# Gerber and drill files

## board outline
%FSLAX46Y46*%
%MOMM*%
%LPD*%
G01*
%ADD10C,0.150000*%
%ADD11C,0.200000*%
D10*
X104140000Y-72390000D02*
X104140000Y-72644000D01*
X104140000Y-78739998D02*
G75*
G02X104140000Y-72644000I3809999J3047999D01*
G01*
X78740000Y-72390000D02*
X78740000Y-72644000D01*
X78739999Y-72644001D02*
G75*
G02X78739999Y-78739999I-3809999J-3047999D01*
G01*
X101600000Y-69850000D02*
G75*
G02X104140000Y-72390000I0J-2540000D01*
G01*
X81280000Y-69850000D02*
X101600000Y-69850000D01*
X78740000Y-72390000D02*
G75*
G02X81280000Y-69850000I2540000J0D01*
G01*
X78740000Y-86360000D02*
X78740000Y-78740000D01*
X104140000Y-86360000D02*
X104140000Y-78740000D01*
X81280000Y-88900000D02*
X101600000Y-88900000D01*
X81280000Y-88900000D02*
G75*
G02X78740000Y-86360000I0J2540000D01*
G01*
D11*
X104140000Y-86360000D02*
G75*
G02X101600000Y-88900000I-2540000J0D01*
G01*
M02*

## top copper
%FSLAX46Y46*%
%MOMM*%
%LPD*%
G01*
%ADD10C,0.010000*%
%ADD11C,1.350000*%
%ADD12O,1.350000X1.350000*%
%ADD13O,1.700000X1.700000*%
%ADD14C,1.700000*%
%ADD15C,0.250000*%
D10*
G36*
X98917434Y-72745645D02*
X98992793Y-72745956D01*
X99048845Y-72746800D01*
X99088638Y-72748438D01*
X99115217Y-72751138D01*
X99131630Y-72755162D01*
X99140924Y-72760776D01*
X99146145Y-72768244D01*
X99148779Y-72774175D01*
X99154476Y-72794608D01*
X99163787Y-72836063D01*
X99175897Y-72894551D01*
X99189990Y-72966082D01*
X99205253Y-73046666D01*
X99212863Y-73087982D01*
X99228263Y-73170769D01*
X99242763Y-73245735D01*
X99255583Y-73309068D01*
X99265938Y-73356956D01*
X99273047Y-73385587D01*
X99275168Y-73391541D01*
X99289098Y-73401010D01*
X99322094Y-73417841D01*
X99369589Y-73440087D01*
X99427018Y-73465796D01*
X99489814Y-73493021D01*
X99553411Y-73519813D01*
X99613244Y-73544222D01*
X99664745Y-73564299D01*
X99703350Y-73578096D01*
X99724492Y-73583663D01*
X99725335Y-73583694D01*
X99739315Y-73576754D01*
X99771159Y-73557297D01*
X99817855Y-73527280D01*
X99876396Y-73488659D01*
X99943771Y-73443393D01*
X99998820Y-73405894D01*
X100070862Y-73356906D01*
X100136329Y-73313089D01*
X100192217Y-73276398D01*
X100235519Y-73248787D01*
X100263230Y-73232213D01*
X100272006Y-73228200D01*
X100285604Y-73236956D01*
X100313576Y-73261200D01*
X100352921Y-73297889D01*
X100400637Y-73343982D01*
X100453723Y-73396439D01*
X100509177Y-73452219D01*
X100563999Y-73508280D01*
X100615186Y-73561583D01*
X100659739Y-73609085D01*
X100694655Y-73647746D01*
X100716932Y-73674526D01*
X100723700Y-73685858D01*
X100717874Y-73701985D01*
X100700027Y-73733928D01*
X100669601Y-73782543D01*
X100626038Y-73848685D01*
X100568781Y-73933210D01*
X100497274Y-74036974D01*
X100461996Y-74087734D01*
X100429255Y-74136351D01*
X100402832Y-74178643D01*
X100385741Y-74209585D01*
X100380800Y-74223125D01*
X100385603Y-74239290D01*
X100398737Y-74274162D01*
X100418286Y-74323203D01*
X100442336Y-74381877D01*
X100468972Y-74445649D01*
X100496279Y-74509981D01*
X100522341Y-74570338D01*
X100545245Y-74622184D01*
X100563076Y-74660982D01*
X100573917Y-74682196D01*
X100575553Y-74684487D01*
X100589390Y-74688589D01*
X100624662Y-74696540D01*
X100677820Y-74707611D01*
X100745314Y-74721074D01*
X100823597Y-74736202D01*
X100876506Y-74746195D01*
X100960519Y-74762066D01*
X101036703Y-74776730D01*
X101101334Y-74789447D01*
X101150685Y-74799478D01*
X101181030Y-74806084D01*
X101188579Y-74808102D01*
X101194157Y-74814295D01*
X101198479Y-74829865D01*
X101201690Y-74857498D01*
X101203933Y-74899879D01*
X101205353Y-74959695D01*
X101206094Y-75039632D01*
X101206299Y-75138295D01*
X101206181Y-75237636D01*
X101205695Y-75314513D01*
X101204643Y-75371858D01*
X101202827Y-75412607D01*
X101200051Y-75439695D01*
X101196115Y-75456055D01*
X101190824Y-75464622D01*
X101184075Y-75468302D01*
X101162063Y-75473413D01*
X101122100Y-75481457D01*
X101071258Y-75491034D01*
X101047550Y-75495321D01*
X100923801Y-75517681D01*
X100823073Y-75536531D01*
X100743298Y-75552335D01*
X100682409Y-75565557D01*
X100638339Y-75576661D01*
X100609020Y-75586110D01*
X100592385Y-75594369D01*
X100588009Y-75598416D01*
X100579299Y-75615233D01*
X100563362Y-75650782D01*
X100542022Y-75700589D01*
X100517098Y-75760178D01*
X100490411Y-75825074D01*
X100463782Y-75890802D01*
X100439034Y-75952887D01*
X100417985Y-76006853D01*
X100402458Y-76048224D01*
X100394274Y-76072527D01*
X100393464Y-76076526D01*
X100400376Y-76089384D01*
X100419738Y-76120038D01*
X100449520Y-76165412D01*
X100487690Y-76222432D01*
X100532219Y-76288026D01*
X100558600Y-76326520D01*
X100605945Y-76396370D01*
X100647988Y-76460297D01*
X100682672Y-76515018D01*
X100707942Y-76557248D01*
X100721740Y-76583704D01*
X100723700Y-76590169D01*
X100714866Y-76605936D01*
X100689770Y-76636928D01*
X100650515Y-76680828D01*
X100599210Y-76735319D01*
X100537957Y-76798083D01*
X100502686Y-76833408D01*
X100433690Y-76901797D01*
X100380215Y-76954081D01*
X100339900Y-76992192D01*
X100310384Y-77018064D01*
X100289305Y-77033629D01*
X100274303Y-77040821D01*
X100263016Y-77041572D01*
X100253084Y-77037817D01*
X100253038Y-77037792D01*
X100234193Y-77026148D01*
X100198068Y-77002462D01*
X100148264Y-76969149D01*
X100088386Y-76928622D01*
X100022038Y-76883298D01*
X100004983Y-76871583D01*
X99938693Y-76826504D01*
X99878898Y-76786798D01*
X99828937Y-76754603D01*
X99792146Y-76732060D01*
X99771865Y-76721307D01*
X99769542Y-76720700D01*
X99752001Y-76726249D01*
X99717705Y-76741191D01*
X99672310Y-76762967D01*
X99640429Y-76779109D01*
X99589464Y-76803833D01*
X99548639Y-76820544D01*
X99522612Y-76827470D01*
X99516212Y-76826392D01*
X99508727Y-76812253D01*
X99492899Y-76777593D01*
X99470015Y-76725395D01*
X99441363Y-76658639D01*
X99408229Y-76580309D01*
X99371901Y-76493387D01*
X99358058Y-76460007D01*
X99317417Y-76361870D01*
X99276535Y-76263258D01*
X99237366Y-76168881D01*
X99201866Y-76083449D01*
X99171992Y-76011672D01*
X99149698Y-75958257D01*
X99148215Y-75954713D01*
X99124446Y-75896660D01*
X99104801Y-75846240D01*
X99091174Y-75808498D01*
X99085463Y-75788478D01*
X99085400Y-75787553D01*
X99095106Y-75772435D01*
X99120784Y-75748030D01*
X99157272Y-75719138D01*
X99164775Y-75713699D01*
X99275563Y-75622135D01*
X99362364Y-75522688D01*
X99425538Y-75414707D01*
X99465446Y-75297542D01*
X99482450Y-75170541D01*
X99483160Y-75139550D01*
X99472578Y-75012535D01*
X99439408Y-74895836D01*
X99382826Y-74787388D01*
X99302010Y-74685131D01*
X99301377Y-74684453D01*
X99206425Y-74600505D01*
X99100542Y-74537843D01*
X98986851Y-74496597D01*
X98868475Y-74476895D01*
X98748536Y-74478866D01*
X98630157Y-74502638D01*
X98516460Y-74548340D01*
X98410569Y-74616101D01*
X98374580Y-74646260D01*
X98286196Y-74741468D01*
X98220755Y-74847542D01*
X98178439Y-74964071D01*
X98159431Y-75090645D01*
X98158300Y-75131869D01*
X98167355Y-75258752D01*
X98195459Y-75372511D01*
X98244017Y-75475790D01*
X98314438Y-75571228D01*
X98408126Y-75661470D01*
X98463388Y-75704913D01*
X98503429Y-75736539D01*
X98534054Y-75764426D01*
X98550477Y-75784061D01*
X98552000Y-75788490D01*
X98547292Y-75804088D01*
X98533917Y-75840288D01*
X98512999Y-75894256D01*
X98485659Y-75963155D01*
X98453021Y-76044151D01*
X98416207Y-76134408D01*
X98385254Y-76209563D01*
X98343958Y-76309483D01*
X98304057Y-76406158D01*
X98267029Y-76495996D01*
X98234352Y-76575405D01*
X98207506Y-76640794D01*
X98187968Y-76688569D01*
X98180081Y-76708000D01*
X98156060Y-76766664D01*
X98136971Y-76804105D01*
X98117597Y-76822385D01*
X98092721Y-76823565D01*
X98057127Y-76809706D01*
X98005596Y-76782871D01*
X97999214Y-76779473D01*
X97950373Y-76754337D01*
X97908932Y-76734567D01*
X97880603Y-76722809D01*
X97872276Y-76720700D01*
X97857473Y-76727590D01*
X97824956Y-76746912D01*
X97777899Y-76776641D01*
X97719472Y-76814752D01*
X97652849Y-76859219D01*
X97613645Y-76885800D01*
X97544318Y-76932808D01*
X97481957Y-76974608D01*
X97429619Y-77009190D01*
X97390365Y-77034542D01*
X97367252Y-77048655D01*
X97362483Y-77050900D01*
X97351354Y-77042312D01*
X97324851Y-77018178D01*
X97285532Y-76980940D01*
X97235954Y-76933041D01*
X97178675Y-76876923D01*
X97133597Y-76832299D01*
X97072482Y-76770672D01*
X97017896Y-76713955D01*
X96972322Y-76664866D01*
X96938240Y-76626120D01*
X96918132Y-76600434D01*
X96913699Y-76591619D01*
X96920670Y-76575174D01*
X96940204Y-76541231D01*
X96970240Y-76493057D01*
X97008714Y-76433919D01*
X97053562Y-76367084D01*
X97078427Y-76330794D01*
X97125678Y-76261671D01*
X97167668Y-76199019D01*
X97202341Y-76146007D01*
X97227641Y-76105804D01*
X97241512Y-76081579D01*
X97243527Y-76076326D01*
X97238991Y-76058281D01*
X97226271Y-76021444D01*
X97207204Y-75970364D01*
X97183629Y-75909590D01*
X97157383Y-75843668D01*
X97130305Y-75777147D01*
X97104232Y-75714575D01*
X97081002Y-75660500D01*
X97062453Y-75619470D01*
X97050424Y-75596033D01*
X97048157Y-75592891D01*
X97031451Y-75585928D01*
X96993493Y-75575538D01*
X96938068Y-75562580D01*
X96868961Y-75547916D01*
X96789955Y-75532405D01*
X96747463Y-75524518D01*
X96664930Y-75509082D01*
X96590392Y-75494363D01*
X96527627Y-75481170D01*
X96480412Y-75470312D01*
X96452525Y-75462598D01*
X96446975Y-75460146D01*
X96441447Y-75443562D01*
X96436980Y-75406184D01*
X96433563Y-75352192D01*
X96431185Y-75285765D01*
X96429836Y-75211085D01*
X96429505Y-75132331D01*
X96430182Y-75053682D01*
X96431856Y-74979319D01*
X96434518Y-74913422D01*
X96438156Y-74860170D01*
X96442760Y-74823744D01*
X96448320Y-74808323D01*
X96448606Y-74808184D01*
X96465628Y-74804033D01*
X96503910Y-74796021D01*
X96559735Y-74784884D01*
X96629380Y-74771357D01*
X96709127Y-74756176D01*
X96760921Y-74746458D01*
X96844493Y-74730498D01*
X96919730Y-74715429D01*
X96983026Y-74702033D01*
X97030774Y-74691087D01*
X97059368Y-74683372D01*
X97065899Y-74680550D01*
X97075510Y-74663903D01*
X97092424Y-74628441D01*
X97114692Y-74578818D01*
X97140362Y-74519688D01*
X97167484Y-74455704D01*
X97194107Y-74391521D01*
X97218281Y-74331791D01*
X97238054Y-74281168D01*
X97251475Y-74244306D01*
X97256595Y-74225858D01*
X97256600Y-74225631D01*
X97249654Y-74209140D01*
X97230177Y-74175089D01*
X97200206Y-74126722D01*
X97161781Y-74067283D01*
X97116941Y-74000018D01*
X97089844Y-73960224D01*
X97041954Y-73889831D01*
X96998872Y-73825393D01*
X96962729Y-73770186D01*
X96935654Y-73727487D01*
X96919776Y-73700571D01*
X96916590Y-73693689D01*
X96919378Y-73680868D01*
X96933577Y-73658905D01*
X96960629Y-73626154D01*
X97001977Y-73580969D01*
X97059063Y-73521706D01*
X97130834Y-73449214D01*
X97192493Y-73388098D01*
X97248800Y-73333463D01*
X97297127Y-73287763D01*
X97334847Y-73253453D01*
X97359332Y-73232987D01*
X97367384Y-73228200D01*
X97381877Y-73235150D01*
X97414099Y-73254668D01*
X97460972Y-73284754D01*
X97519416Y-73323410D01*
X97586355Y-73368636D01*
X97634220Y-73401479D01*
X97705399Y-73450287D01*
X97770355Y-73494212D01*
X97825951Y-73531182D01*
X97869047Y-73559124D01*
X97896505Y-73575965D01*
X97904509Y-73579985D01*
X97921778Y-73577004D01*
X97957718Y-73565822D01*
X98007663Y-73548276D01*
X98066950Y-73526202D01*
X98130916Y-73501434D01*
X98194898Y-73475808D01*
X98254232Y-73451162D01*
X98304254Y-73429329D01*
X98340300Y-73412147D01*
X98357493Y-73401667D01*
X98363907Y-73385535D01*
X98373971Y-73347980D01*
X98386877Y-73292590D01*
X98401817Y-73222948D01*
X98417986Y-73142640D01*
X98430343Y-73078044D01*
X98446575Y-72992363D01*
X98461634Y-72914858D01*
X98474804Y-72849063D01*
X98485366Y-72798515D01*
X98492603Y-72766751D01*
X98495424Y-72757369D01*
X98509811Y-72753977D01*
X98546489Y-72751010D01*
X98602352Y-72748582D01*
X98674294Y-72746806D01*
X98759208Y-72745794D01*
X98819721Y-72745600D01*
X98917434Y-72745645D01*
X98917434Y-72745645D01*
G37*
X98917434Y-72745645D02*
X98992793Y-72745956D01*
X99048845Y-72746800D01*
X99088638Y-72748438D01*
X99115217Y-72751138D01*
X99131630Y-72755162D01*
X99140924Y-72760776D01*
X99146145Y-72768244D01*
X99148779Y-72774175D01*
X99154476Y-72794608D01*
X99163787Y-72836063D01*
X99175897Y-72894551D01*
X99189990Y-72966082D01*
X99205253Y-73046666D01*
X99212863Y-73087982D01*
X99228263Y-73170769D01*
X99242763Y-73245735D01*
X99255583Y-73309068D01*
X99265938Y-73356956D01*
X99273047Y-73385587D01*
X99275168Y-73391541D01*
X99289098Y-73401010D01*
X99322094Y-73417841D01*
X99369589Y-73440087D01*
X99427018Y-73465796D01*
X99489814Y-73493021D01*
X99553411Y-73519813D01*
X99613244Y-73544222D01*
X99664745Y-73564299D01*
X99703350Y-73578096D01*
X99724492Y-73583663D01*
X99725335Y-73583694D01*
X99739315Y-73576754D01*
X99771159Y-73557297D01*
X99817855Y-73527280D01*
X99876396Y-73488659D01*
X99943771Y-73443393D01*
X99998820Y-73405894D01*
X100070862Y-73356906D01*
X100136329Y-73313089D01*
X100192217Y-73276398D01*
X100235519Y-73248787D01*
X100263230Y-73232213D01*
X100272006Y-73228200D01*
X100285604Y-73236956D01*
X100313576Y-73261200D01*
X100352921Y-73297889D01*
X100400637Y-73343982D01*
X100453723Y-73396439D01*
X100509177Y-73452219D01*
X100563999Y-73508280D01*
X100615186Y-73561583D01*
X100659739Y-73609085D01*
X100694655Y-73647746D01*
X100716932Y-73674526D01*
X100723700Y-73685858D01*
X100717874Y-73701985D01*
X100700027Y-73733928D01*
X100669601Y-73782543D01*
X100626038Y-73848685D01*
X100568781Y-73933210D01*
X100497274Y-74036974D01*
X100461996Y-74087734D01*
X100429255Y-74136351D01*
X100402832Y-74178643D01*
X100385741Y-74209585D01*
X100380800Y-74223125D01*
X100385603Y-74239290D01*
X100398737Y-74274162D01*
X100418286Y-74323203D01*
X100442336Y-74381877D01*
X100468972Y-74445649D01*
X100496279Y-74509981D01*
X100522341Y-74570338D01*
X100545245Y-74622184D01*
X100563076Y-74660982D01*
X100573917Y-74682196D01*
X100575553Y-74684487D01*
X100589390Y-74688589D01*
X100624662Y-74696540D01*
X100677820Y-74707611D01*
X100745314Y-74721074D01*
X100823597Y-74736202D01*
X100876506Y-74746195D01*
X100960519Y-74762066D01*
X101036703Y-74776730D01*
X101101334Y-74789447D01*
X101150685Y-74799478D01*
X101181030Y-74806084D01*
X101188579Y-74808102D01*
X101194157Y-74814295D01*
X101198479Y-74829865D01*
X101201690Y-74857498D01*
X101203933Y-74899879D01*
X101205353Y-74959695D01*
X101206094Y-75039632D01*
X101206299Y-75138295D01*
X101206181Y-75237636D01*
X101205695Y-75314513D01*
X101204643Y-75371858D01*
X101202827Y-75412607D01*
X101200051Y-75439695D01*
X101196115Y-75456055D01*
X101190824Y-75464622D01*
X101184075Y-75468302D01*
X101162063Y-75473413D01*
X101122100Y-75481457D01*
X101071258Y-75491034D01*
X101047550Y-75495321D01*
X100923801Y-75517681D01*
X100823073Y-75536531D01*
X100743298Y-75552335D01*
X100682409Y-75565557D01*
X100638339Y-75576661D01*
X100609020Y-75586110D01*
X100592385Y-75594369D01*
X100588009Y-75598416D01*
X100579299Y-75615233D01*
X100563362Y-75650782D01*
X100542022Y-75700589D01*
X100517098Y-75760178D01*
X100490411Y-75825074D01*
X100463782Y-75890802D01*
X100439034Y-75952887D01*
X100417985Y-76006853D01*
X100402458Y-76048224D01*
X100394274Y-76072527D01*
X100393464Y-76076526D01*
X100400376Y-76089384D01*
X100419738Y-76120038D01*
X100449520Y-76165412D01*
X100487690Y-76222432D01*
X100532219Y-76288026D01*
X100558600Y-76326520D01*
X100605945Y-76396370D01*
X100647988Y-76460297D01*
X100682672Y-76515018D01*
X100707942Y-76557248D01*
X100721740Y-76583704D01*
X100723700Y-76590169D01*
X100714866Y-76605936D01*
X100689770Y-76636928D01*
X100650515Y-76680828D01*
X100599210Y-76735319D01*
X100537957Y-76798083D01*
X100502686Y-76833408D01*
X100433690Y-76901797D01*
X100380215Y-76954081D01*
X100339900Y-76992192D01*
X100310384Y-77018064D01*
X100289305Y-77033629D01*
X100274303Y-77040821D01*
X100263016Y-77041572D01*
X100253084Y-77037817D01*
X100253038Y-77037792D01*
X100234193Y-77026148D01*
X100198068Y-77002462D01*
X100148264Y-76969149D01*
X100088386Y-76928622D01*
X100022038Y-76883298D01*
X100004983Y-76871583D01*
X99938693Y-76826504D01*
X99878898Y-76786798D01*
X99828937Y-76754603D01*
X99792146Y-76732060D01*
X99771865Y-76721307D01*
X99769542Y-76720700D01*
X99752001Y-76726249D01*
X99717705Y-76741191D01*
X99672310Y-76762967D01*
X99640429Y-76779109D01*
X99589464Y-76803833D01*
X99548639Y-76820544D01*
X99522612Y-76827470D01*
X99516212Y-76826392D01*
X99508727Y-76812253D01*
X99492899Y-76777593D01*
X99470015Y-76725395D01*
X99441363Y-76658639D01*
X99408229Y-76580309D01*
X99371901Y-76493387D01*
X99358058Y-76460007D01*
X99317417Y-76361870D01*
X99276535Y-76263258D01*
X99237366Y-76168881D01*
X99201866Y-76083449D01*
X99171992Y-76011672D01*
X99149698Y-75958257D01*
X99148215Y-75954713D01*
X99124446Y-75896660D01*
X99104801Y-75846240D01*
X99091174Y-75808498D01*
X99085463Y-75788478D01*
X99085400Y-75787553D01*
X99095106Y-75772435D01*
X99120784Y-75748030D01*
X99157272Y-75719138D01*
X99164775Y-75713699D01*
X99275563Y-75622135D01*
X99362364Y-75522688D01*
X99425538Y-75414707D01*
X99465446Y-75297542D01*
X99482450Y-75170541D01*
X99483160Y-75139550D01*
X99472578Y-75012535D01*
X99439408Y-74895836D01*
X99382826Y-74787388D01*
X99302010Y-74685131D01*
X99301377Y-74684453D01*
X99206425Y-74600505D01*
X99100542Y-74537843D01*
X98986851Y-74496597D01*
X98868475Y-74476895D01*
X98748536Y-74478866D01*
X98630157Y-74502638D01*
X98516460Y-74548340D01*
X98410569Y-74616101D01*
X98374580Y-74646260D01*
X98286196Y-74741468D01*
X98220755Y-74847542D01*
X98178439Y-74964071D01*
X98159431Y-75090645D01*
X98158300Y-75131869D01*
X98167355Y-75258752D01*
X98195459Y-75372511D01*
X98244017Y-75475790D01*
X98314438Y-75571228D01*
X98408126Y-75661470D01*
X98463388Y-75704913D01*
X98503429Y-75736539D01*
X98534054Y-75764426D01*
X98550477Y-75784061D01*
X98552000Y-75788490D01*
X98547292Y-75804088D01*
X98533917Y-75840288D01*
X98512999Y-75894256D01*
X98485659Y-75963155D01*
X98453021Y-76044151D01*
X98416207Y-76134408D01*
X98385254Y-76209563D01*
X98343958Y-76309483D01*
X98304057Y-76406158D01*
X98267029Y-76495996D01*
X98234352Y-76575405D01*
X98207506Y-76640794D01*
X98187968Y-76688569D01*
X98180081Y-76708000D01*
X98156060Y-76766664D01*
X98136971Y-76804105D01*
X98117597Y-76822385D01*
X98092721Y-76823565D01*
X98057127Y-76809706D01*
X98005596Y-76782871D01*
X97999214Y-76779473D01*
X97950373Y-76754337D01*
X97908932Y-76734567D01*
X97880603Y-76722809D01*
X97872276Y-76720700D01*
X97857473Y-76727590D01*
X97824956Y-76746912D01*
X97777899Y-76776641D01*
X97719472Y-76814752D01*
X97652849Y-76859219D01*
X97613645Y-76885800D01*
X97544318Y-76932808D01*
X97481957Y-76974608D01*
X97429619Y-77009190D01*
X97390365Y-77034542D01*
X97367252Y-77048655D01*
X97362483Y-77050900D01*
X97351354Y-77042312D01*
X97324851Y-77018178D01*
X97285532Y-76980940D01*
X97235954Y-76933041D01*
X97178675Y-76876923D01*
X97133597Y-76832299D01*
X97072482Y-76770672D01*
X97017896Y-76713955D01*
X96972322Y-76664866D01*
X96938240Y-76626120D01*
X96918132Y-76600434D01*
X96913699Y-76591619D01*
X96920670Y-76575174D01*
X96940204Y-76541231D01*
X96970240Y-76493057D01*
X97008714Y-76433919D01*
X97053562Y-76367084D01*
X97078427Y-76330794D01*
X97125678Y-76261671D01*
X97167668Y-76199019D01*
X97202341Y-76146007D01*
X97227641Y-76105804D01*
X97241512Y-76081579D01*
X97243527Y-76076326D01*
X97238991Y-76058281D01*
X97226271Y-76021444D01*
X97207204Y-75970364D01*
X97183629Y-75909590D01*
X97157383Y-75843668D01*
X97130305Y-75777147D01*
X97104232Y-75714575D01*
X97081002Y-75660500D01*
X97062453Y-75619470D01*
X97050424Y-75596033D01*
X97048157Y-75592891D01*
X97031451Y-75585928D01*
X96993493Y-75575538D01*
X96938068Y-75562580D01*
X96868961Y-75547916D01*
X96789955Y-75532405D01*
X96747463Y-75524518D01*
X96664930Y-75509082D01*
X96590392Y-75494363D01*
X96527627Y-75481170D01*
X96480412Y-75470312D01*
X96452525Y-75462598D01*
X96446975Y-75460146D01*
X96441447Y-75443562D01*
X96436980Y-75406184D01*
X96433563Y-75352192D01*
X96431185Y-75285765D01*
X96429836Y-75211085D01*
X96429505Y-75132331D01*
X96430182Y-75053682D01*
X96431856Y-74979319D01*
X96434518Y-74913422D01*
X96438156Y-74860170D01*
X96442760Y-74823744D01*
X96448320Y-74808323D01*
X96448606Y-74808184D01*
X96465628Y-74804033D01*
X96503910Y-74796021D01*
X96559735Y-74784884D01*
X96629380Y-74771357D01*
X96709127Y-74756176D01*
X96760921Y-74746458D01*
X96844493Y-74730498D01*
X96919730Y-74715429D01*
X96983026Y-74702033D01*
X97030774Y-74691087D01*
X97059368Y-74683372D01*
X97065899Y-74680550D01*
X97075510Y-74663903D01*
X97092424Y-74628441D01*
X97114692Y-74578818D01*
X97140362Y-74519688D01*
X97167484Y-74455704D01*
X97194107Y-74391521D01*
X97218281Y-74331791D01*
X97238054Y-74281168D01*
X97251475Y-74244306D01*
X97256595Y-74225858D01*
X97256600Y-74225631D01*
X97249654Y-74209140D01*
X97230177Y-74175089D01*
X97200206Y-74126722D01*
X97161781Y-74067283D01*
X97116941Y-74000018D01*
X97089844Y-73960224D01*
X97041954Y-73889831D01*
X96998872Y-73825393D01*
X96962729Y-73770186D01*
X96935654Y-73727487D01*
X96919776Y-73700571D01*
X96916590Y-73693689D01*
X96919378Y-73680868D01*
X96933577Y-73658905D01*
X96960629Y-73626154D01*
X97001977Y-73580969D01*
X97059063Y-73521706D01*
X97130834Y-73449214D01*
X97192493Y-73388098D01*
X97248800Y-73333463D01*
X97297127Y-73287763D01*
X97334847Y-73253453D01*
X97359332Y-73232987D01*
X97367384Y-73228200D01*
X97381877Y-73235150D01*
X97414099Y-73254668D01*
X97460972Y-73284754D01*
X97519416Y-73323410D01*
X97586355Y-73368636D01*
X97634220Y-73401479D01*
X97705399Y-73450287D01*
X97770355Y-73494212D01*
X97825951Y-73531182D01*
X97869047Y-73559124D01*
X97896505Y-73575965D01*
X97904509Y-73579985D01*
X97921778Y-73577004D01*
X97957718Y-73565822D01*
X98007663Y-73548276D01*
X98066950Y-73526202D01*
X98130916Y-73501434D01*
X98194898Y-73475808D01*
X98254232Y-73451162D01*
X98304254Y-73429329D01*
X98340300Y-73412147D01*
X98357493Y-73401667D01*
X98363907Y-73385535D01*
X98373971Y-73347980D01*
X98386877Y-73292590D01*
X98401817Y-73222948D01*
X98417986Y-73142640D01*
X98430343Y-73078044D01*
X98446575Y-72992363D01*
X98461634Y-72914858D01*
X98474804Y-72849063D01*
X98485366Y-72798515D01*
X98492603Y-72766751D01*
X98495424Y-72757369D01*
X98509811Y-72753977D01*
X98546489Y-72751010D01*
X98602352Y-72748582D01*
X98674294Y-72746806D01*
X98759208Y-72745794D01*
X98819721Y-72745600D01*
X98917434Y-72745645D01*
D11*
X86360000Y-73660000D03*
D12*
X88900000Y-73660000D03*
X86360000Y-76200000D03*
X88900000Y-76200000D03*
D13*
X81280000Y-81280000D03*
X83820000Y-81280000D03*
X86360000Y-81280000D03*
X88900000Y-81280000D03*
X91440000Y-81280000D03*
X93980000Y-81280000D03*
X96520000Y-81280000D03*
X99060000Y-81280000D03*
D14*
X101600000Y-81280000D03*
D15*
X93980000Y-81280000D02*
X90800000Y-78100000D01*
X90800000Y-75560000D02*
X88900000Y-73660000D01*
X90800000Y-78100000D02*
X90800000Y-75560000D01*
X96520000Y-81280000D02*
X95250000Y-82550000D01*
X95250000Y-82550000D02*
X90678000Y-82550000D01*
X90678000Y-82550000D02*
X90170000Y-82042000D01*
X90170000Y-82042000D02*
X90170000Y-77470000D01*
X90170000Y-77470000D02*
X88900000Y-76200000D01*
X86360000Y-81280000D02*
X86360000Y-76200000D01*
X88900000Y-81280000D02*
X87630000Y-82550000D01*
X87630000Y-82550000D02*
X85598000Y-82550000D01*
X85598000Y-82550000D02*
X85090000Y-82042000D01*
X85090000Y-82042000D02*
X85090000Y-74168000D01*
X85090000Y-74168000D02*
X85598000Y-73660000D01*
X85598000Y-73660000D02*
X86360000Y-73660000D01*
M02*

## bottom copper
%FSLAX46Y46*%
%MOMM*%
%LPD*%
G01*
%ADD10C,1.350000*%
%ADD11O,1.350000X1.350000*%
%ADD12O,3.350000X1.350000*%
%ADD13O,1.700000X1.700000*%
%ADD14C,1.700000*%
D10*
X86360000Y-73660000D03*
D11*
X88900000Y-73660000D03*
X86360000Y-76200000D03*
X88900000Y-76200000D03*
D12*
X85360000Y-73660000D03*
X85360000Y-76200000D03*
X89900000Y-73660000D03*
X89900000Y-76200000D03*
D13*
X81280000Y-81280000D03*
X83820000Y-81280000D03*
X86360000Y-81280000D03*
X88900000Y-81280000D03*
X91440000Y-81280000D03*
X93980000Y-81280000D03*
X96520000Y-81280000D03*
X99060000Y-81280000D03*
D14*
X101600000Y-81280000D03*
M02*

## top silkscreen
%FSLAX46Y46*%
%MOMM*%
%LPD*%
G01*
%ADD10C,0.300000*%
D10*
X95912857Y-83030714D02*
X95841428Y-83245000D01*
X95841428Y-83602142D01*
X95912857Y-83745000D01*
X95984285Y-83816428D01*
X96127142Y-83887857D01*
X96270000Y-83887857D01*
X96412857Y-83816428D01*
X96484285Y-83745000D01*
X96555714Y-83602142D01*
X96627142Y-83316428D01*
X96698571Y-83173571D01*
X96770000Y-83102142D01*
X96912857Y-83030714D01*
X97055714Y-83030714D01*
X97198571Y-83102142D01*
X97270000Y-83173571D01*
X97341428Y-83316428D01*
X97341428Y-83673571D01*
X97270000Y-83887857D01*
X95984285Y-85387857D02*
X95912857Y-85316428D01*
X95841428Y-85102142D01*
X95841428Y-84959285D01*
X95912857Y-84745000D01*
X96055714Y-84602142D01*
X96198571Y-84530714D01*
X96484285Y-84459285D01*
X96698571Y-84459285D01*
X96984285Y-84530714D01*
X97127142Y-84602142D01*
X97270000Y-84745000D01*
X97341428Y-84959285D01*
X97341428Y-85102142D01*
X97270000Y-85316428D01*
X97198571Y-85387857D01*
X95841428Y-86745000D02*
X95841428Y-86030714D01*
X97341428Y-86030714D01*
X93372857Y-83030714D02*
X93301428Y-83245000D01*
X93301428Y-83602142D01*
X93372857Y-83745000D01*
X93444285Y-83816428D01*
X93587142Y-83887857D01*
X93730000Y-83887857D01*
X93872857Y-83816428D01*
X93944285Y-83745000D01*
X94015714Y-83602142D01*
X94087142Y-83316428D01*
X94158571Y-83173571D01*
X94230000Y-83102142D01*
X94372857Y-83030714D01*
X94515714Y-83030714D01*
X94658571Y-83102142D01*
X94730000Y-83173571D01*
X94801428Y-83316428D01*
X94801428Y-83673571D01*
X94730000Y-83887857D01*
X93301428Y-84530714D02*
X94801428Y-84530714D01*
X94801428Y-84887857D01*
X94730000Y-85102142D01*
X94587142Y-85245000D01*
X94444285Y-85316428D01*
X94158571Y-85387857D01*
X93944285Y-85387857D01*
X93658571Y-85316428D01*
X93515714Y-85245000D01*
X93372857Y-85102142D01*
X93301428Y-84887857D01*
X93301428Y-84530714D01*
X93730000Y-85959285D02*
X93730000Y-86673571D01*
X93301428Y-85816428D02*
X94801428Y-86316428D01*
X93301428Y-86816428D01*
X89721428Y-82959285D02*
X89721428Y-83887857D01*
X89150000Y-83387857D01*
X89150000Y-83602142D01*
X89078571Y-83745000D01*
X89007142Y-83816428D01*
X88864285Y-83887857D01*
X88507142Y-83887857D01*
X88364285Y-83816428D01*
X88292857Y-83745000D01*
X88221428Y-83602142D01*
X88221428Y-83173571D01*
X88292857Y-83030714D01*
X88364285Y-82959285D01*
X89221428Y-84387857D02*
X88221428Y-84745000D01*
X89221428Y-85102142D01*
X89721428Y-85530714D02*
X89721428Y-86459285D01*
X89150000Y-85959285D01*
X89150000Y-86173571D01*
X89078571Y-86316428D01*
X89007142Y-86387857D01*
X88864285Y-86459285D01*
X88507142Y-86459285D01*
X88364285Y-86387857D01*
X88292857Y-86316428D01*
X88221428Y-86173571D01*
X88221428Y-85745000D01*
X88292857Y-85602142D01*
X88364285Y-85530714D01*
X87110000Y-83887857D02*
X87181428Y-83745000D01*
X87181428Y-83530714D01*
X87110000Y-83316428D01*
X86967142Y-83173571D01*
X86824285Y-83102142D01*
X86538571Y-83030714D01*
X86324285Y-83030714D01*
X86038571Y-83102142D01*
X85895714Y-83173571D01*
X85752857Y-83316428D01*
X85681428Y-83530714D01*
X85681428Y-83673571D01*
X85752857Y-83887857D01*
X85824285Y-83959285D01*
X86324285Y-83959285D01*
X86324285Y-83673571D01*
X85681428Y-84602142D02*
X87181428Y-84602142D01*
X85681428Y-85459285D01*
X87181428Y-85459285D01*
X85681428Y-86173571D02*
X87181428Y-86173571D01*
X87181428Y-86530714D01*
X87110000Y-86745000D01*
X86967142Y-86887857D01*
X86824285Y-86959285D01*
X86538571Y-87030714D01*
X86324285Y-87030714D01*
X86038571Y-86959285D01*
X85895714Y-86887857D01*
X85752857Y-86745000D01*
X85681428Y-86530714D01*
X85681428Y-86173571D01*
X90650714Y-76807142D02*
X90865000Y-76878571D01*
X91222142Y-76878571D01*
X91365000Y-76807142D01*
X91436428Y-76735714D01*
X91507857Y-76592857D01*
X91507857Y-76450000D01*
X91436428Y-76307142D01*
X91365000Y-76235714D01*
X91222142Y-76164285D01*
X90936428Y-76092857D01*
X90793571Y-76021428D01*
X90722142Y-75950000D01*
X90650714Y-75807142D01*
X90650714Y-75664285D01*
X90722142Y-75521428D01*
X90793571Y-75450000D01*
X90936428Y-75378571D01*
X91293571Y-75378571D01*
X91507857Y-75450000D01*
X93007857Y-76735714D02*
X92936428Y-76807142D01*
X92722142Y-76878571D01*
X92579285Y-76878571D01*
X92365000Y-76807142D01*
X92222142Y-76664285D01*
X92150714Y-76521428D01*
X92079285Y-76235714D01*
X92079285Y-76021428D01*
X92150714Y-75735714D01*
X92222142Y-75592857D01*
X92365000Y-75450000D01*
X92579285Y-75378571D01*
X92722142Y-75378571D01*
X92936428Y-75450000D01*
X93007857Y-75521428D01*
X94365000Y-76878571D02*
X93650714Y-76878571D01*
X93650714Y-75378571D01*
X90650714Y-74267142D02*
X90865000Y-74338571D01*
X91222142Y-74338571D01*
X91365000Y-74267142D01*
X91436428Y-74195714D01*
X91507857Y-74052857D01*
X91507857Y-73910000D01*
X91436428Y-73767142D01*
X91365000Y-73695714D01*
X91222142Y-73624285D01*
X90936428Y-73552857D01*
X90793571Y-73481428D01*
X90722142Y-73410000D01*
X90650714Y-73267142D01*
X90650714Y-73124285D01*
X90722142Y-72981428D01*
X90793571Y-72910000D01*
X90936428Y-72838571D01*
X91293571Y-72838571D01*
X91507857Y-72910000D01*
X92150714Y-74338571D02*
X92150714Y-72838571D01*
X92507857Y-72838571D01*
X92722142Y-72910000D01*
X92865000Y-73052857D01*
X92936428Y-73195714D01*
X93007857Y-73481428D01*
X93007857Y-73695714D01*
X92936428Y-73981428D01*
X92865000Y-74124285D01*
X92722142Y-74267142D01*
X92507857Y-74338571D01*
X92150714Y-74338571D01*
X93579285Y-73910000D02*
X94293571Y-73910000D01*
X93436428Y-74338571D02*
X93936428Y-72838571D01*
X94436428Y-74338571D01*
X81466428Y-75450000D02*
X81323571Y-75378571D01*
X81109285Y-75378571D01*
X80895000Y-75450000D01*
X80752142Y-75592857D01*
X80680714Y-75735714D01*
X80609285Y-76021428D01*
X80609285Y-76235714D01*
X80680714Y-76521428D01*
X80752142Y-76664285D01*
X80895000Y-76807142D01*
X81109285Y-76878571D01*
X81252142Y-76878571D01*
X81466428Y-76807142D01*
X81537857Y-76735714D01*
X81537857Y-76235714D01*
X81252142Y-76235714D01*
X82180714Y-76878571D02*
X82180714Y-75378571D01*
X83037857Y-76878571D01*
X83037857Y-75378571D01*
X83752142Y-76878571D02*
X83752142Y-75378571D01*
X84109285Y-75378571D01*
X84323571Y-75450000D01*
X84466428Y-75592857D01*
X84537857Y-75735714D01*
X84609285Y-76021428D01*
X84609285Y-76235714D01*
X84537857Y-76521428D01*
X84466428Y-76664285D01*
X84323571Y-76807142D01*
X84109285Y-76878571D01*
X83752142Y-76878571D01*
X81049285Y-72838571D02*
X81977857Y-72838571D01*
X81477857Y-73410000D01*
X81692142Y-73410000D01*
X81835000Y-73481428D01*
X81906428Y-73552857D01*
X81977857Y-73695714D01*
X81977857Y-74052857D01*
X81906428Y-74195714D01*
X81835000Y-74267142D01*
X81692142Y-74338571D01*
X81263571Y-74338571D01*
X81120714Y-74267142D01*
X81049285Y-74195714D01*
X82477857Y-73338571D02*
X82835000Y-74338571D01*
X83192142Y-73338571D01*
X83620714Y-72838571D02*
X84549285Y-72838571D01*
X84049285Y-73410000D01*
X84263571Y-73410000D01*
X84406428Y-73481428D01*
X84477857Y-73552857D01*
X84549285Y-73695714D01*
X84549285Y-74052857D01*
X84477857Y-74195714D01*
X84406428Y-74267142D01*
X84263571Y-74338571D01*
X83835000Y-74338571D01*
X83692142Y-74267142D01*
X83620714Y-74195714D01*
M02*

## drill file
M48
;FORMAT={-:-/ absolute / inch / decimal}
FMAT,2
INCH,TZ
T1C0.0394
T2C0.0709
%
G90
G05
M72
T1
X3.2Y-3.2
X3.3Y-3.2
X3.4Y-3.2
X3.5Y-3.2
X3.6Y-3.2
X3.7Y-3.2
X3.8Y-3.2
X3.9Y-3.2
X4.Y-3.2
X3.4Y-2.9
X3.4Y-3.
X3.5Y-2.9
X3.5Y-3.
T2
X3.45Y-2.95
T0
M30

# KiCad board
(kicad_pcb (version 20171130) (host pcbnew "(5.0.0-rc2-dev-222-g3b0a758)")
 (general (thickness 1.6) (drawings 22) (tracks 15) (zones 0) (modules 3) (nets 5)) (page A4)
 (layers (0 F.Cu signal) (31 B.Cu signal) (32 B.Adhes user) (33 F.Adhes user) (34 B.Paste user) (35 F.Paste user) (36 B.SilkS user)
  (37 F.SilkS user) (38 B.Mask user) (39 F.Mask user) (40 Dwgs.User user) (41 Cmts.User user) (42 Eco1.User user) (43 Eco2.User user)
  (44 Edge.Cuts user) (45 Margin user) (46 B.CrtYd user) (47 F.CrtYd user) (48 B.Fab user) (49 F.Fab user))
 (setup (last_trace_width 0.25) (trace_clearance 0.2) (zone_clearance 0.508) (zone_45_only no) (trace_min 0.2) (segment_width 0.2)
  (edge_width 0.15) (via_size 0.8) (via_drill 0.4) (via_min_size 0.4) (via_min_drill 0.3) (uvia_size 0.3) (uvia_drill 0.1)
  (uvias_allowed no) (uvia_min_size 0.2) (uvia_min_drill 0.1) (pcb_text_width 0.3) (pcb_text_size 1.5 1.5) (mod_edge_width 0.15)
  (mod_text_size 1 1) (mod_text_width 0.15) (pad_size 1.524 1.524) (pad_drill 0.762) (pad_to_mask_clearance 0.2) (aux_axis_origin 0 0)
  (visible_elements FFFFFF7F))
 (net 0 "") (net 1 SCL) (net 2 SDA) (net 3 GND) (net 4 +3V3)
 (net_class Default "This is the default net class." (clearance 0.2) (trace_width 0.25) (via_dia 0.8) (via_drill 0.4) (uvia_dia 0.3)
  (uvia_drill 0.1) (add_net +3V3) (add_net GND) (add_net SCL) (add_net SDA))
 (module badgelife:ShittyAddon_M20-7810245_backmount (layer F.Cu) (at 86.36 73.66)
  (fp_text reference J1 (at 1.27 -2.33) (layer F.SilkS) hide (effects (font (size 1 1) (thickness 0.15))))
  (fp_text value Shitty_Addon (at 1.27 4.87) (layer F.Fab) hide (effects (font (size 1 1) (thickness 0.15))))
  (pad "" np_thru_hole circle (at 1.27 1.27) (size 1.8 1.8) (drill 1.8) (layers *.Cu *.Mask) (solder_mask_margin 0.001))
  (pad 3 smd oval (at 2.54 2.54) (size 3.35 1.35) (drill (offset 1 0)) (layers B.Cu B.Paste B.Mask) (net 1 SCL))
  (pad 4 smd oval (at 2.54 0) (size 3.35 1.35) (drill (offset 1 0)) (layers B.Cu B.Paste B.Mask) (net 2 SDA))
  (pad 2 smd oval (at 0 2.54) (size 3.35 1.35) (drill (offset -1 0)) (layers B.Cu B.Paste B.Mask) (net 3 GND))
  (pad 1 smd oval (at 0 0) (size 3.35 1.35) (drill (offset -1 0)) (layers B.Cu B.Paste B.Mask) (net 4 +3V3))
  (pad 3 thru_hole oval (at 2.54 2.54) (size 1.35 1.35) (drill 1) (layers *.Cu *.Mask) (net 1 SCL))
  (pad 2 thru_hole oval (at 0 2.54) (size 1.35 1.35) (drill 1) (layers *.Cu *.Mask) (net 3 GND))
  (pad 4 thru_hole oval (at 2.54 0) (size 1.35 1.35) (drill 1) (layers *.Cu *.Mask) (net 2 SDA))
  (pad 1 thru_hole circle (at 0 0) (size 1.35 1.35) (drill 1) (layers *.Cu *.Mask) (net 4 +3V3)))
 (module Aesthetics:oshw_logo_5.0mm (layer F.Cu) (at 98.806 74.93)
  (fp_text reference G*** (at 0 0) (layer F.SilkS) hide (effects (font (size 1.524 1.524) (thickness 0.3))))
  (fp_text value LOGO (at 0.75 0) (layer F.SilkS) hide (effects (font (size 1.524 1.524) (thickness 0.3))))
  (fp_poly
   (pts (xy 0.111434 -2.184355) (xy 0.186793 -2.184044) (xy 0.242845 -2.1832) (xy 0.282638 -2.181562) (xy 0.309217 -2.178862)
    (xy 0.32563 -2.174838) (xy 0.334924 -2.169224) (xy 0.340145 -2.161756) (xy 0.342779 -2.155825) (xy 0.348476 -2.135392)
    (xy 0.357787 -2.093937) (xy 0.369897 -2.035449) (xy 0.38399 -1.963918) (xy 0.399253 -1.883334) (xy 0.406863 -1.842018)
    (xy 0.422263 -1.759231) (xy 0.436763 -1.684265) (xy 0.449583 -1.620932) (xy 0.459938 -1.573044) (xy 0.467047 -1.544413)
    (xy 0.469168 -1.538459) (xy 0.483098 -1.52899) (xy 0.516094 -1.512159) (xy 0.563589 -1.489913) (xy 0.621018 -1.464204)
    (xy 0.683814 -1.436979) (xy 0.747411 -1.410187) (xy 0.807244 -1.385778) (xy 0.858745 -1.365701) (xy 0.89735 -1.351904)
    (xy 0.918492 -1.346337) (xy 0.919335 -1.346306) (xy 0.933315 -1.353246) (xy 0.965159 -1.372703) (xy 1.011855 -1.40272)
    (xy 1.070396 -1.441341) (xy 1.137771 -1.486607) (xy 1.19282 -1.524106) (xy 1.264862 -1.573094) (xy 1.330329 -1.616911)
    (xy 1.386217 -1.653602) (xy 1.429519 -1.681213) (xy 1.45723 -1.697787) (xy 1.466006 -1.7018) (xy 1.479604 -1.693044)
    (xy 1.507576 -1.6688) (xy 1.546921 -1.632111) (xy 1.594637 -1.586018) (xy 1.647723 -1.533561) (xy 1.703177 -1.477781)
    (xy 1.757999 -1.42172) (xy 1.809186 -1.368417) (xy 1.853739 -1.320915) (xy 1.888655 -1.282254) (xy 1.910932 -1.255474)
    (xy 1.9177 -1.244142) (xy 1.911874 -1.228015) (xy 1.894027 -1.196072) (xy 1.863601 -1.147457) (xy 1.820038 -1.081315)
    (xy 1.762781 -0.99679) (xy 1.691274 -0.893026) (xy 1.655996 -0.842266) (xy 1.623255 -0.793649) (xy 1.596832 -0.751357)
    (xy 1.579741 -0.720415) (xy 1.5748 -0.706875) (xy 1.579603 -0.69071) (xy 1.592737 -0.655838) (xy 1.612286 -0.606797)
    (xy 1.636336 -0.548123) (xy 1.662972 -0.484351) (xy 1.690279 -0.420019) (xy 1.716341 -0.359662) (xy 1.739245 -0.307816)
    (xy 1.757076 -0.269018) (xy 1.767917 -0.247804) (xy 1.769553 -0.245513) (xy 1.78339 -0.241411) (xy 1.818662 -0.23346)
    (xy 1.87182 -0.222389) (xy 1.939314 -0.208926) (xy 2.017597 -0.193798) (xy 2.070506 -0.183805) (xy 2.154519 -0.167934)
    (xy 2.230703 -0.15327) (xy 2.295334 -0.140553) (xy 2.344685 -0.130522) (xy 2.37503 -0.123916) (xy 2.382579 -0.121898)
    (xy 2.388157 -0.115705) (xy 2.392479 -0.100135) (xy 2.39569 -0.072502) (xy 2.397933 -0.030121) (xy 2.399353 0.029695)
    (xy 2.400094 0.109632) (xy 2.400299 0.208295) (xy 2.400181 0.307636) (xy 2.399695 0.384513) (xy 2.398643 0.441858)
    (xy 2.396827 0.482607) (xy 2.394051 0.509695) (xy 2.390115 0.526055) (xy 2.384824 0.534622) (xy 2.378075 0.538302)
    (xy 2.356063 0.543413) (xy 2.3161 0.551457) (xy 2.265258 0.561034) (xy 2.24155 0.565321) (xy 2.117801 0.587681) (xy 2.017073 0.606531)
    (xy 1.937298 0.622335) (xy 1.876409 0.635557) (xy 1.832339 0.646661) (xy 1.80302 0.65611) (xy 1.786385 0.664369) (xy 1.782009 0.668416)
    (xy 1.773299 0.685233) (xy 1.757362 0.720782) (xy 1.736022 0.770589) (xy 1.711098 0.830178) (xy 1.684411 0.895074)
    (xy 1.657782 0.960802) (xy 1.633034 1.022887) (xy 1.611985 1.076853) (xy 1.596458 1.118224) (xy 1.588274 1.142527)
    (xy 1.587464 1.146526) (xy 1.594376 1.159384) (xy 1.613738 1.190038) (xy 1.64352 1.235412) (xy 1.68169 1.292432) (xy 1.726219 1.358026)
    (xy 1.7526 1.39652) (xy 1.799945 1.46637) (xy 1.841988 1.530297) (xy 1.876672 1.585018) (xy 1.901942 1.627248) (xy 1.91574 1.653704)
    (xy 1.9177 1.660169) (xy 1.908866 1.675936) (xy 1.88377 1.706928) (xy 1.844515 1.750828) (xy 1.79321 1.805319) (xy 1.731957 1.868083)
    (xy 1.696686 1.903408) (xy 1.62769 1.971797) (xy 1.574215 2.024081) (xy 1.5339 2.062192) (xy 1.504384 2.088064) (xy 1.483305 2.103629)
    (xy 1.468303 2.110821) (xy 1.457016 2.111572) (xy 1.447084 2.107817) (xy 1.447038 2.107792) (xy 1.428193 2.096148)
    (xy 1.392068 2.072462) (xy 1.342264 2.039149) (xy 1.282386 1.998622) (xy 1.216038 1.953298) (xy 1.198983 1.941583)
    (xy 1.132693 1.896504) (xy 1.072898 1.856798) (xy 1.022937 1.824603) (xy 0.986146 1.80206) (xy 0.965865 1.791307) (xy 0.963542 1.7907)
    (xy 0.946001 1.796249) (xy 0.911705 1.811191) (xy 0.86631 1.832967) (xy 0.834429 1.849109) (xy 0.783464 1.873833) (xy 0.742639 1.890544)
    (xy 0.716612 1.89747) (xy 0.710212 1.896392) (xy 0.702727 1.882253) (xy 0.686899 1.847593) (xy 0.664015 1.795395) (xy 0.635363 1.728639)
    (xy 0.602229 1.650309) (xy 0.565901 1.563387) (xy 0.552058 1.530007) (xy 0.511417 1.43187) (xy 0.470535 1.333258) (xy 0.431366 1.238881)
    (xy 0.395866 1.153449) (xy 0.365992 1.081672) (xy 0.343698 1.028257) (xy 0.342215 1.024713) (xy 0.318446 0.96666) (xy 0.298801 0.91624)
    (xy 0.285174 0.878498) (xy 0.279463 0.858478) (xy 0.2794 0.857553) (xy 0.289106 0.842435) (xy 0.314784 0.81803) (xy 0.351272 0.789138)
    (xy 0.358775 0.783699) (xy 0.469563 0.692135) (xy 0.556364 0.592688) (xy 0.619538 0.484707) (xy 0.659446 0.367542) (xy 0.67645 0.240541)
    (xy 0.67716 0.20955) (xy 0.666578 0.082535) (xy 0.633408 -0.034164) (xy 0.576826 -0.142612) (xy 0.49601 -0.244869)
    (xy 0.495377 -0.245547) (xy 0.400425 -0.329495) (xy 0.294542 -0.392157) (xy 0.180851 -0.433403) (xy 0.062475 -0.453105)
    (xy -0.057464 -0.451134) (xy -0.175843 -0.427362) (xy -0.28954 -0.38166) (xy -0.395431 -0.313899) (xy -0.43142 -0.28374)
    (xy -0.519804 -0.188532) (xy -0.585245 -0.082458) (xy -0.627561 0.034071) (xy -0.646569 0.160645) (xy -0.6477 0.201869)
    (xy -0.638645 0.328752) (xy -0.610541 0.442511) (xy -0.561983 0.54579) (xy -0.491562 0.641228) (xy -0.397874 0.73147)
    (xy -0.342612 0.774913) (xy -0.302571 0.806539) (xy -0.271946 0.834426) (xy -0.255523 0.854061) (xy -0.254 0.85849)
    (xy -0.258708 0.874088) (xy -0.272083 0.910288) (xy -0.293001 0.964256) (xy -0.320341 1.033155) (xy -0.352979 1.114151)
    (xy -0.389793 1.204408) (xy -0.420746 1.279563) (xy -0.462042 1.379483) (xy -0.501943 1.476158) (xy -0.538971 1.565996)
    (xy -0.571648 1.645405) (xy -0.598494 1.710794) (xy -0.618032 1.758569) (xy -0.625919 1.778) (xy -0.64994 1.836664)
    (xy -0.669029 1.874105) (xy -0.688403 1.892385) (xy -0.713279 1.893565) (xy -0.748873 1.879706) (xy -0.800404 1.852871)
    (xy -0.806786 1.849473) (xy -0.855627 1.824337) (xy -0.897068 1.804567) (xy -0.925397 1.792809) (xy -0.933724 1.7907)
    (xy -0.948527 1.79759) (xy -0.981044 1.816912) (xy -1.028101 1.846641) (xy -1.086528 1.884752) (xy -1.153151 1.929219)
    (xy -1.192355 1.9558) (xy -1.261682 2.002808) (xy -1.324043 2.044608) (xy -1.376381 2.07919) (xy -1.415635 2.104542)
    (xy -1.438748 2.118655) (xy -1.443517 2.1209) (xy -1.454646 2.112312) (xy -1.481149 2.088178) (xy -1.520468 2.05094)
    (xy -1.570046 2.003041) (xy -1.627325 1.946923) (xy -1.672403 1.902299) (xy -1.733518 1.840672) (xy -1.788104 1.783955)
    (xy -1.833678 1.734866) (xy -1.86776 1.69612) (xy -1.887868 1.670434) (xy -1.892301 1.661619) (xy -1.88533 1.645174)
    (xy -1.865796 1.611231) (xy -1.83576 1.563057) (xy -1.797286 1.503919) (xy -1.752438 1.437084) (xy -1.727573 1.400794)
    (xy -1.680322 1.331671) (xy -1.638332 1.269019) (xy -1.603659 1.216007) (xy -1.578359 1.175804) (xy -1.564488 1.151579)
    (xy -1.562473 1.146326) (xy -1.567009 1.128281) (xy -1.579729 1.091444) (xy -1.598796 1.040364) (xy -1.622371 0.97959)
    (xy -1.648617 0.913668) (xy -1.675695 0.847147) (xy -1.701768 0.784575) (xy -1.724998 0.7305) (xy -1.743547 0.68947)
    (xy -1.755576 0.666033) (xy -1.757843 0.662891) (xy -1.774549 0.655928) (xy -1.812507 0.645538) (xy -1.867932 0.63258)
    (xy -1.937039 0.617916) (xy -2.016045 0.602405) (xy -2.058537 0.594518) (xy -2.14107 0.579082) (xy -2.215608 0.564363)
    (xy -2.278373 0.55117) (xy -2.325588 0.540312) (xy -2.353475 0.532598) (xy -2.359025 0.530146) (xy -2.364553 0.513562)
    (xy -2.36902 0.476184) (xy -2.372437 0.422192) (xy -2.374815 0.355765) (xy -2.376164 0.281085) (xy -2.376495 0.202331)
    (xy -2.375818 0.123682) (xy -2.374144 0.049319) (xy -2.371482 -0.016578) (xy -2.367844 -0.06983) (xy -2.36324 -0.106256)
    (xy -2.35768 -0.121677) (xy -2.357394 -0.121816) (xy -2.340372 -0.125967) (xy -2.30209 -0.133979) (xy -2.246265 -0.145116)
    (xy -2.17662 -0.158643) (xy -2.096873 -0.173824) (xy -2.045079 -0.183542) (xy -1.961507 -0.199502) (xy -1.88627 -0.214571)
    (xy -1.822974 -0.227967) (xy -1.775226 -0.238913) (xy -1.746632 -0.246628) (xy -1.740101 -0.24945) (xy -1.73049 -0.266097)
    (xy -1.713576 -0.301559) (xy -1.691308 -0.351182) (xy -1.665638 -0.410312) (xy -1.638516 -0.474296) (xy -1.611893 -0.538479)
    (xy -1.587719 -0.598209) (xy -1.567946 -0.648832) (xy -1.554525 -0.685694) (xy -1.549405 -0.704142) (xy -1.5494 -0.704369)
    (xy -1.556346 -0.72086) (xy -1.575823 -0.754911) (xy -1.605794 -0.803278) (xy -1.644219 -0.862717) (xy -1.689059 -0.929982)
    (xy -1.716156 -0.969776) (xy -1.764046 -1.040169) (xy -1.807128 -1.104607) (xy -1.843271 -1.159814) (xy -1.870346 -1.202513)
    (xy -1.886224 -1.229429) (xy -1.88941 -1.236311) (xy -1.886622 -1.249132) (xy -1.872423 -1.271095) (xy -1.845371 -1.303846)
    (xy -1.804023 -1.349031) (xy -1.746937 -1.408294) (xy -1.675166 -1.480786) (xy -1.613507 -1.541902) (xy -1.5572 -1.596537)
    (xy -1.508873 -1.642237) (xy -1.471153 -1.676547) (xy -1.446668 -1.697013) (xy -1.438616 -1.7018) (xy -1.424123 -1.69485)
    (xy -1.391901 -1.675332) (xy -1.345028 -1.645246) (xy -1.286584 -1.60659) (xy -1.219645 -1.561364) (xy -1.17178 -1.528521)
    (xy -1.100601 -1.479713) (xy -1.035645 -1.435788) (xy -0.980049 -1.398818) (xy -0.936953 -1.370876) (xy -0.909495 -1.354035)
    (xy -0.901491 -1.350015) (xy -0.884222 -1.352996) (xy -0.848282 -1.364178) (xy -0.798337 -1.381724) (xy -0.73905 -1.403798)
    (xy -0.675084 -1.428566) (xy -0.611102 -1.454192) (xy -0.551768 -1.478838) (xy -0.501746 -1.500671) (xy -0.4657 -1.517853)
    (xy -0.448507 -1.528333) (xy -0.442093 -1.544465) (xy -0.432029 -1.58202) (xy -0.419123 -1.63741) (xy -0.404183 -1.707052)
    (xy -0.388014 -1.78736) (xy -0.375657 -1.851956) (xy -0.359425 -1.937637) (xy -0.344366 -2.015142) (xy -0.331196 -2.080937)
    (xy -0.320634 -2.131485) (xy -0.313397 -2.163249) (xy -0.310576 -2.172631) (xy -0.296189 -2.176023) (xy -0.259511 -2.17899)
    (xy -0.203648 -2.181418) (xy -0.131706 -2.183194) (xy -0.046792 -2.184206) (xy 0.013721 -2.1844) (xy 0.111434 -2.184355))
   (layer F.Cu) (width 0.01)))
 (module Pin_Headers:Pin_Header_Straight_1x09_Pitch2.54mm (layer F.Cu) (at 101.6 81.28 270)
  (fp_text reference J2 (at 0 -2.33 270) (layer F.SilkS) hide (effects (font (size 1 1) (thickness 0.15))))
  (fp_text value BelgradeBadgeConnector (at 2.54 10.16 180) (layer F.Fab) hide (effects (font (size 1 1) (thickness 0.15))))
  (pad 9 thru_hole oval (at 0 20.32 270) (size 1.7 1.7) (drill 1) (layers *.Cu *.Mask))
  (pad 8 thru_hole oval (at 0 17.78 270) (size 1.7 1.7) (drill 1) (layers *.Cu *.Mask))
  (pad 7 thru_hole oval (at 0 15.24 270) (size 1.7 1.7) (drill 1) (layers *.Cu *.Mask) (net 3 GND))
  (pad 6 thru_hole oval (at 0 12.7 270) (size 1.7 1.7) (drill 1) (layers *.Cu *.Mask) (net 4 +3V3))
  (pad 5 thru_hole oval (at 0 10.16 270) (size 1.7 1.7) (drill 1) (layers *.Cu *.Mask))
  (pad 4 thru_hole oval (at 0 7.62 270) (size 1.7 1.7) (drill 1) (layers *.Cu *.Mask) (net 2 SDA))
  (pad 3 thru_hole oval (at 0 5.08 270) (size 1.7 1.7) (drill 1) (layers *.Cu *.Mask) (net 1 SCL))
  (pad 2 thru_hole oval (at 0 2.54 270) (size 1.7 1.7) (drill 1) (layers *.Cu *.Mask))
  (pad 1 thru_hole circle (at 0 0 270) (size 1.7 1.7) (drill 1) (layers *.Cu *.Mask)))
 (gr_line (start 104.14 72.39) (end 104.14 72.644) (layer Edge.Cuts) (width 0.15))
 (gr_arc (start 107.949999 75.691999) (end 104.14 72.644) (angle -77.31961651) (layer Edge.Cuts) (width 0.15))
 (gr_line (start 78.74 72.39) (end 78.74 72.644) (layer Edge.Cuts) (width 0.15))
 (gr_arc (start 74.93 75.692) (end 78.739999 78.739999) (angle -77.31961651) (layer Edge.Cuts) (width 0.15))
 (gr_arc (start 101.6 72.39) (end 104.14 72.39) (angle -90) (layer Edge.Cuts) (width 0.15))
 (gr_line (start 81.28 69.85) (end 101.6 69.85) (layer Edge.Cuts) (width 0.15))
 (gr_arc (start 81.28 72.39) (end 81.28 69.85) (angle -90) (layer Edge.Cuts) (width 0.15))
 (gr_line (start 78.74 86.36) (end 78.74 78.74) (layer Edge.Cuts) (width 0.15))
 (gr_line (start 104.14 86.36) (end 104.14 78.74) (layer Edge.Cuts) (width 0.15))
 (gr_line (start 81.28 88.9) (end 101.6 88.9) (layer Edge.Cuts) (width 0.15))
 (gr_arc (start 81.28 86.36) (end 78.74 86.36) (angle -90) (layer Edge.Cuts) (width 0.15))
 (gr_arc (start 101.6 86.36) (end 101.6 88.9) (angle -90) (layer Edge.Cuts) (width 0.2))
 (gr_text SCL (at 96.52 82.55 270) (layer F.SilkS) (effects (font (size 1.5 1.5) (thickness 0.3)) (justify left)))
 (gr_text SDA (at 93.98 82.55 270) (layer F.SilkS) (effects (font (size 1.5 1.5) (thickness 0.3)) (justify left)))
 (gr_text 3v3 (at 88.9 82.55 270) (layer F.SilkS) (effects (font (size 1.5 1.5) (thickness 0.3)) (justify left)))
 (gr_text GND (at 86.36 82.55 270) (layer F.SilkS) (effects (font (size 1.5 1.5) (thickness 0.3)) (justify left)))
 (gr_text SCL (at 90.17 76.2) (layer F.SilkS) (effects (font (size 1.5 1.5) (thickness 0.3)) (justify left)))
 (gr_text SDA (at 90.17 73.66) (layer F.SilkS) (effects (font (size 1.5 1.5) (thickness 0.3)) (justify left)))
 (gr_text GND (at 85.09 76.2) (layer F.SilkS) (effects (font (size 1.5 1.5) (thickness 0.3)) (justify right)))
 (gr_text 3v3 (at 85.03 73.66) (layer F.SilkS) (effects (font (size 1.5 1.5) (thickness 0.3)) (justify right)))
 (segment (start 93.98 81.28) (end 90.8 78.1) (width 0.25) (layer F.Cu) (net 2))
 (segment (start 90.8 75.56) (end 88.9 73.66) (width 0.25) (layer F.Cu) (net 2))
 (segment (start 90.8 78.1) (end 90.8 75.56) (width 0.25) (layer F.Cu) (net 2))
 (segment (start 96.52 81.28) (end 95.25 82.55) (width 0.25) (layer F.Cu) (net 1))
 (segment (start 95.25 82.55) (end 90.678 82.55) (width 0.25) (layer F.Cu) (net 1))
 (segment (start 90.678 82.55) (end 90.17 82.042) (width 0.25) (layer F.Cu) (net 1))
 (segment (start 90.17 82.042) (end 90.17 77.47) (width 0.25) (layer F.Cu) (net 1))
 (segment (start 90.17 77.47) (end 88.9 76.2) (width 0.25) (layer F.Cu) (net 1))
 (segment (start 86.36 81.28) (end 86.36 76.2) (width 0.25) (layer F.Cu) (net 3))
 (segment (start 88.9 81.28) (end 87.63 82.55) (width 0.25) (layer F.Cu) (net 4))
 (segment (start 87.63 82.55) (end 85.598 82.55) (width 0.25) (layer F.Cu) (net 4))
 (segment (start 85.598 82.55) (end 85.09 82.042) (width 0.25) (layer F.Cu) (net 4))
 (segment (start 85.09 82.042) (end 85.09 74.168) (width 0.25) (layer F.Cu) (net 4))
 (segment (start 85.09 74.168) (end 85.598 73.66) (width 0.25) (layer F.Cu) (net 4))
 (segment (start 85.598 73.66) (end 86.36 73.66) (width 0.25) (layer F.Cu) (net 4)))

